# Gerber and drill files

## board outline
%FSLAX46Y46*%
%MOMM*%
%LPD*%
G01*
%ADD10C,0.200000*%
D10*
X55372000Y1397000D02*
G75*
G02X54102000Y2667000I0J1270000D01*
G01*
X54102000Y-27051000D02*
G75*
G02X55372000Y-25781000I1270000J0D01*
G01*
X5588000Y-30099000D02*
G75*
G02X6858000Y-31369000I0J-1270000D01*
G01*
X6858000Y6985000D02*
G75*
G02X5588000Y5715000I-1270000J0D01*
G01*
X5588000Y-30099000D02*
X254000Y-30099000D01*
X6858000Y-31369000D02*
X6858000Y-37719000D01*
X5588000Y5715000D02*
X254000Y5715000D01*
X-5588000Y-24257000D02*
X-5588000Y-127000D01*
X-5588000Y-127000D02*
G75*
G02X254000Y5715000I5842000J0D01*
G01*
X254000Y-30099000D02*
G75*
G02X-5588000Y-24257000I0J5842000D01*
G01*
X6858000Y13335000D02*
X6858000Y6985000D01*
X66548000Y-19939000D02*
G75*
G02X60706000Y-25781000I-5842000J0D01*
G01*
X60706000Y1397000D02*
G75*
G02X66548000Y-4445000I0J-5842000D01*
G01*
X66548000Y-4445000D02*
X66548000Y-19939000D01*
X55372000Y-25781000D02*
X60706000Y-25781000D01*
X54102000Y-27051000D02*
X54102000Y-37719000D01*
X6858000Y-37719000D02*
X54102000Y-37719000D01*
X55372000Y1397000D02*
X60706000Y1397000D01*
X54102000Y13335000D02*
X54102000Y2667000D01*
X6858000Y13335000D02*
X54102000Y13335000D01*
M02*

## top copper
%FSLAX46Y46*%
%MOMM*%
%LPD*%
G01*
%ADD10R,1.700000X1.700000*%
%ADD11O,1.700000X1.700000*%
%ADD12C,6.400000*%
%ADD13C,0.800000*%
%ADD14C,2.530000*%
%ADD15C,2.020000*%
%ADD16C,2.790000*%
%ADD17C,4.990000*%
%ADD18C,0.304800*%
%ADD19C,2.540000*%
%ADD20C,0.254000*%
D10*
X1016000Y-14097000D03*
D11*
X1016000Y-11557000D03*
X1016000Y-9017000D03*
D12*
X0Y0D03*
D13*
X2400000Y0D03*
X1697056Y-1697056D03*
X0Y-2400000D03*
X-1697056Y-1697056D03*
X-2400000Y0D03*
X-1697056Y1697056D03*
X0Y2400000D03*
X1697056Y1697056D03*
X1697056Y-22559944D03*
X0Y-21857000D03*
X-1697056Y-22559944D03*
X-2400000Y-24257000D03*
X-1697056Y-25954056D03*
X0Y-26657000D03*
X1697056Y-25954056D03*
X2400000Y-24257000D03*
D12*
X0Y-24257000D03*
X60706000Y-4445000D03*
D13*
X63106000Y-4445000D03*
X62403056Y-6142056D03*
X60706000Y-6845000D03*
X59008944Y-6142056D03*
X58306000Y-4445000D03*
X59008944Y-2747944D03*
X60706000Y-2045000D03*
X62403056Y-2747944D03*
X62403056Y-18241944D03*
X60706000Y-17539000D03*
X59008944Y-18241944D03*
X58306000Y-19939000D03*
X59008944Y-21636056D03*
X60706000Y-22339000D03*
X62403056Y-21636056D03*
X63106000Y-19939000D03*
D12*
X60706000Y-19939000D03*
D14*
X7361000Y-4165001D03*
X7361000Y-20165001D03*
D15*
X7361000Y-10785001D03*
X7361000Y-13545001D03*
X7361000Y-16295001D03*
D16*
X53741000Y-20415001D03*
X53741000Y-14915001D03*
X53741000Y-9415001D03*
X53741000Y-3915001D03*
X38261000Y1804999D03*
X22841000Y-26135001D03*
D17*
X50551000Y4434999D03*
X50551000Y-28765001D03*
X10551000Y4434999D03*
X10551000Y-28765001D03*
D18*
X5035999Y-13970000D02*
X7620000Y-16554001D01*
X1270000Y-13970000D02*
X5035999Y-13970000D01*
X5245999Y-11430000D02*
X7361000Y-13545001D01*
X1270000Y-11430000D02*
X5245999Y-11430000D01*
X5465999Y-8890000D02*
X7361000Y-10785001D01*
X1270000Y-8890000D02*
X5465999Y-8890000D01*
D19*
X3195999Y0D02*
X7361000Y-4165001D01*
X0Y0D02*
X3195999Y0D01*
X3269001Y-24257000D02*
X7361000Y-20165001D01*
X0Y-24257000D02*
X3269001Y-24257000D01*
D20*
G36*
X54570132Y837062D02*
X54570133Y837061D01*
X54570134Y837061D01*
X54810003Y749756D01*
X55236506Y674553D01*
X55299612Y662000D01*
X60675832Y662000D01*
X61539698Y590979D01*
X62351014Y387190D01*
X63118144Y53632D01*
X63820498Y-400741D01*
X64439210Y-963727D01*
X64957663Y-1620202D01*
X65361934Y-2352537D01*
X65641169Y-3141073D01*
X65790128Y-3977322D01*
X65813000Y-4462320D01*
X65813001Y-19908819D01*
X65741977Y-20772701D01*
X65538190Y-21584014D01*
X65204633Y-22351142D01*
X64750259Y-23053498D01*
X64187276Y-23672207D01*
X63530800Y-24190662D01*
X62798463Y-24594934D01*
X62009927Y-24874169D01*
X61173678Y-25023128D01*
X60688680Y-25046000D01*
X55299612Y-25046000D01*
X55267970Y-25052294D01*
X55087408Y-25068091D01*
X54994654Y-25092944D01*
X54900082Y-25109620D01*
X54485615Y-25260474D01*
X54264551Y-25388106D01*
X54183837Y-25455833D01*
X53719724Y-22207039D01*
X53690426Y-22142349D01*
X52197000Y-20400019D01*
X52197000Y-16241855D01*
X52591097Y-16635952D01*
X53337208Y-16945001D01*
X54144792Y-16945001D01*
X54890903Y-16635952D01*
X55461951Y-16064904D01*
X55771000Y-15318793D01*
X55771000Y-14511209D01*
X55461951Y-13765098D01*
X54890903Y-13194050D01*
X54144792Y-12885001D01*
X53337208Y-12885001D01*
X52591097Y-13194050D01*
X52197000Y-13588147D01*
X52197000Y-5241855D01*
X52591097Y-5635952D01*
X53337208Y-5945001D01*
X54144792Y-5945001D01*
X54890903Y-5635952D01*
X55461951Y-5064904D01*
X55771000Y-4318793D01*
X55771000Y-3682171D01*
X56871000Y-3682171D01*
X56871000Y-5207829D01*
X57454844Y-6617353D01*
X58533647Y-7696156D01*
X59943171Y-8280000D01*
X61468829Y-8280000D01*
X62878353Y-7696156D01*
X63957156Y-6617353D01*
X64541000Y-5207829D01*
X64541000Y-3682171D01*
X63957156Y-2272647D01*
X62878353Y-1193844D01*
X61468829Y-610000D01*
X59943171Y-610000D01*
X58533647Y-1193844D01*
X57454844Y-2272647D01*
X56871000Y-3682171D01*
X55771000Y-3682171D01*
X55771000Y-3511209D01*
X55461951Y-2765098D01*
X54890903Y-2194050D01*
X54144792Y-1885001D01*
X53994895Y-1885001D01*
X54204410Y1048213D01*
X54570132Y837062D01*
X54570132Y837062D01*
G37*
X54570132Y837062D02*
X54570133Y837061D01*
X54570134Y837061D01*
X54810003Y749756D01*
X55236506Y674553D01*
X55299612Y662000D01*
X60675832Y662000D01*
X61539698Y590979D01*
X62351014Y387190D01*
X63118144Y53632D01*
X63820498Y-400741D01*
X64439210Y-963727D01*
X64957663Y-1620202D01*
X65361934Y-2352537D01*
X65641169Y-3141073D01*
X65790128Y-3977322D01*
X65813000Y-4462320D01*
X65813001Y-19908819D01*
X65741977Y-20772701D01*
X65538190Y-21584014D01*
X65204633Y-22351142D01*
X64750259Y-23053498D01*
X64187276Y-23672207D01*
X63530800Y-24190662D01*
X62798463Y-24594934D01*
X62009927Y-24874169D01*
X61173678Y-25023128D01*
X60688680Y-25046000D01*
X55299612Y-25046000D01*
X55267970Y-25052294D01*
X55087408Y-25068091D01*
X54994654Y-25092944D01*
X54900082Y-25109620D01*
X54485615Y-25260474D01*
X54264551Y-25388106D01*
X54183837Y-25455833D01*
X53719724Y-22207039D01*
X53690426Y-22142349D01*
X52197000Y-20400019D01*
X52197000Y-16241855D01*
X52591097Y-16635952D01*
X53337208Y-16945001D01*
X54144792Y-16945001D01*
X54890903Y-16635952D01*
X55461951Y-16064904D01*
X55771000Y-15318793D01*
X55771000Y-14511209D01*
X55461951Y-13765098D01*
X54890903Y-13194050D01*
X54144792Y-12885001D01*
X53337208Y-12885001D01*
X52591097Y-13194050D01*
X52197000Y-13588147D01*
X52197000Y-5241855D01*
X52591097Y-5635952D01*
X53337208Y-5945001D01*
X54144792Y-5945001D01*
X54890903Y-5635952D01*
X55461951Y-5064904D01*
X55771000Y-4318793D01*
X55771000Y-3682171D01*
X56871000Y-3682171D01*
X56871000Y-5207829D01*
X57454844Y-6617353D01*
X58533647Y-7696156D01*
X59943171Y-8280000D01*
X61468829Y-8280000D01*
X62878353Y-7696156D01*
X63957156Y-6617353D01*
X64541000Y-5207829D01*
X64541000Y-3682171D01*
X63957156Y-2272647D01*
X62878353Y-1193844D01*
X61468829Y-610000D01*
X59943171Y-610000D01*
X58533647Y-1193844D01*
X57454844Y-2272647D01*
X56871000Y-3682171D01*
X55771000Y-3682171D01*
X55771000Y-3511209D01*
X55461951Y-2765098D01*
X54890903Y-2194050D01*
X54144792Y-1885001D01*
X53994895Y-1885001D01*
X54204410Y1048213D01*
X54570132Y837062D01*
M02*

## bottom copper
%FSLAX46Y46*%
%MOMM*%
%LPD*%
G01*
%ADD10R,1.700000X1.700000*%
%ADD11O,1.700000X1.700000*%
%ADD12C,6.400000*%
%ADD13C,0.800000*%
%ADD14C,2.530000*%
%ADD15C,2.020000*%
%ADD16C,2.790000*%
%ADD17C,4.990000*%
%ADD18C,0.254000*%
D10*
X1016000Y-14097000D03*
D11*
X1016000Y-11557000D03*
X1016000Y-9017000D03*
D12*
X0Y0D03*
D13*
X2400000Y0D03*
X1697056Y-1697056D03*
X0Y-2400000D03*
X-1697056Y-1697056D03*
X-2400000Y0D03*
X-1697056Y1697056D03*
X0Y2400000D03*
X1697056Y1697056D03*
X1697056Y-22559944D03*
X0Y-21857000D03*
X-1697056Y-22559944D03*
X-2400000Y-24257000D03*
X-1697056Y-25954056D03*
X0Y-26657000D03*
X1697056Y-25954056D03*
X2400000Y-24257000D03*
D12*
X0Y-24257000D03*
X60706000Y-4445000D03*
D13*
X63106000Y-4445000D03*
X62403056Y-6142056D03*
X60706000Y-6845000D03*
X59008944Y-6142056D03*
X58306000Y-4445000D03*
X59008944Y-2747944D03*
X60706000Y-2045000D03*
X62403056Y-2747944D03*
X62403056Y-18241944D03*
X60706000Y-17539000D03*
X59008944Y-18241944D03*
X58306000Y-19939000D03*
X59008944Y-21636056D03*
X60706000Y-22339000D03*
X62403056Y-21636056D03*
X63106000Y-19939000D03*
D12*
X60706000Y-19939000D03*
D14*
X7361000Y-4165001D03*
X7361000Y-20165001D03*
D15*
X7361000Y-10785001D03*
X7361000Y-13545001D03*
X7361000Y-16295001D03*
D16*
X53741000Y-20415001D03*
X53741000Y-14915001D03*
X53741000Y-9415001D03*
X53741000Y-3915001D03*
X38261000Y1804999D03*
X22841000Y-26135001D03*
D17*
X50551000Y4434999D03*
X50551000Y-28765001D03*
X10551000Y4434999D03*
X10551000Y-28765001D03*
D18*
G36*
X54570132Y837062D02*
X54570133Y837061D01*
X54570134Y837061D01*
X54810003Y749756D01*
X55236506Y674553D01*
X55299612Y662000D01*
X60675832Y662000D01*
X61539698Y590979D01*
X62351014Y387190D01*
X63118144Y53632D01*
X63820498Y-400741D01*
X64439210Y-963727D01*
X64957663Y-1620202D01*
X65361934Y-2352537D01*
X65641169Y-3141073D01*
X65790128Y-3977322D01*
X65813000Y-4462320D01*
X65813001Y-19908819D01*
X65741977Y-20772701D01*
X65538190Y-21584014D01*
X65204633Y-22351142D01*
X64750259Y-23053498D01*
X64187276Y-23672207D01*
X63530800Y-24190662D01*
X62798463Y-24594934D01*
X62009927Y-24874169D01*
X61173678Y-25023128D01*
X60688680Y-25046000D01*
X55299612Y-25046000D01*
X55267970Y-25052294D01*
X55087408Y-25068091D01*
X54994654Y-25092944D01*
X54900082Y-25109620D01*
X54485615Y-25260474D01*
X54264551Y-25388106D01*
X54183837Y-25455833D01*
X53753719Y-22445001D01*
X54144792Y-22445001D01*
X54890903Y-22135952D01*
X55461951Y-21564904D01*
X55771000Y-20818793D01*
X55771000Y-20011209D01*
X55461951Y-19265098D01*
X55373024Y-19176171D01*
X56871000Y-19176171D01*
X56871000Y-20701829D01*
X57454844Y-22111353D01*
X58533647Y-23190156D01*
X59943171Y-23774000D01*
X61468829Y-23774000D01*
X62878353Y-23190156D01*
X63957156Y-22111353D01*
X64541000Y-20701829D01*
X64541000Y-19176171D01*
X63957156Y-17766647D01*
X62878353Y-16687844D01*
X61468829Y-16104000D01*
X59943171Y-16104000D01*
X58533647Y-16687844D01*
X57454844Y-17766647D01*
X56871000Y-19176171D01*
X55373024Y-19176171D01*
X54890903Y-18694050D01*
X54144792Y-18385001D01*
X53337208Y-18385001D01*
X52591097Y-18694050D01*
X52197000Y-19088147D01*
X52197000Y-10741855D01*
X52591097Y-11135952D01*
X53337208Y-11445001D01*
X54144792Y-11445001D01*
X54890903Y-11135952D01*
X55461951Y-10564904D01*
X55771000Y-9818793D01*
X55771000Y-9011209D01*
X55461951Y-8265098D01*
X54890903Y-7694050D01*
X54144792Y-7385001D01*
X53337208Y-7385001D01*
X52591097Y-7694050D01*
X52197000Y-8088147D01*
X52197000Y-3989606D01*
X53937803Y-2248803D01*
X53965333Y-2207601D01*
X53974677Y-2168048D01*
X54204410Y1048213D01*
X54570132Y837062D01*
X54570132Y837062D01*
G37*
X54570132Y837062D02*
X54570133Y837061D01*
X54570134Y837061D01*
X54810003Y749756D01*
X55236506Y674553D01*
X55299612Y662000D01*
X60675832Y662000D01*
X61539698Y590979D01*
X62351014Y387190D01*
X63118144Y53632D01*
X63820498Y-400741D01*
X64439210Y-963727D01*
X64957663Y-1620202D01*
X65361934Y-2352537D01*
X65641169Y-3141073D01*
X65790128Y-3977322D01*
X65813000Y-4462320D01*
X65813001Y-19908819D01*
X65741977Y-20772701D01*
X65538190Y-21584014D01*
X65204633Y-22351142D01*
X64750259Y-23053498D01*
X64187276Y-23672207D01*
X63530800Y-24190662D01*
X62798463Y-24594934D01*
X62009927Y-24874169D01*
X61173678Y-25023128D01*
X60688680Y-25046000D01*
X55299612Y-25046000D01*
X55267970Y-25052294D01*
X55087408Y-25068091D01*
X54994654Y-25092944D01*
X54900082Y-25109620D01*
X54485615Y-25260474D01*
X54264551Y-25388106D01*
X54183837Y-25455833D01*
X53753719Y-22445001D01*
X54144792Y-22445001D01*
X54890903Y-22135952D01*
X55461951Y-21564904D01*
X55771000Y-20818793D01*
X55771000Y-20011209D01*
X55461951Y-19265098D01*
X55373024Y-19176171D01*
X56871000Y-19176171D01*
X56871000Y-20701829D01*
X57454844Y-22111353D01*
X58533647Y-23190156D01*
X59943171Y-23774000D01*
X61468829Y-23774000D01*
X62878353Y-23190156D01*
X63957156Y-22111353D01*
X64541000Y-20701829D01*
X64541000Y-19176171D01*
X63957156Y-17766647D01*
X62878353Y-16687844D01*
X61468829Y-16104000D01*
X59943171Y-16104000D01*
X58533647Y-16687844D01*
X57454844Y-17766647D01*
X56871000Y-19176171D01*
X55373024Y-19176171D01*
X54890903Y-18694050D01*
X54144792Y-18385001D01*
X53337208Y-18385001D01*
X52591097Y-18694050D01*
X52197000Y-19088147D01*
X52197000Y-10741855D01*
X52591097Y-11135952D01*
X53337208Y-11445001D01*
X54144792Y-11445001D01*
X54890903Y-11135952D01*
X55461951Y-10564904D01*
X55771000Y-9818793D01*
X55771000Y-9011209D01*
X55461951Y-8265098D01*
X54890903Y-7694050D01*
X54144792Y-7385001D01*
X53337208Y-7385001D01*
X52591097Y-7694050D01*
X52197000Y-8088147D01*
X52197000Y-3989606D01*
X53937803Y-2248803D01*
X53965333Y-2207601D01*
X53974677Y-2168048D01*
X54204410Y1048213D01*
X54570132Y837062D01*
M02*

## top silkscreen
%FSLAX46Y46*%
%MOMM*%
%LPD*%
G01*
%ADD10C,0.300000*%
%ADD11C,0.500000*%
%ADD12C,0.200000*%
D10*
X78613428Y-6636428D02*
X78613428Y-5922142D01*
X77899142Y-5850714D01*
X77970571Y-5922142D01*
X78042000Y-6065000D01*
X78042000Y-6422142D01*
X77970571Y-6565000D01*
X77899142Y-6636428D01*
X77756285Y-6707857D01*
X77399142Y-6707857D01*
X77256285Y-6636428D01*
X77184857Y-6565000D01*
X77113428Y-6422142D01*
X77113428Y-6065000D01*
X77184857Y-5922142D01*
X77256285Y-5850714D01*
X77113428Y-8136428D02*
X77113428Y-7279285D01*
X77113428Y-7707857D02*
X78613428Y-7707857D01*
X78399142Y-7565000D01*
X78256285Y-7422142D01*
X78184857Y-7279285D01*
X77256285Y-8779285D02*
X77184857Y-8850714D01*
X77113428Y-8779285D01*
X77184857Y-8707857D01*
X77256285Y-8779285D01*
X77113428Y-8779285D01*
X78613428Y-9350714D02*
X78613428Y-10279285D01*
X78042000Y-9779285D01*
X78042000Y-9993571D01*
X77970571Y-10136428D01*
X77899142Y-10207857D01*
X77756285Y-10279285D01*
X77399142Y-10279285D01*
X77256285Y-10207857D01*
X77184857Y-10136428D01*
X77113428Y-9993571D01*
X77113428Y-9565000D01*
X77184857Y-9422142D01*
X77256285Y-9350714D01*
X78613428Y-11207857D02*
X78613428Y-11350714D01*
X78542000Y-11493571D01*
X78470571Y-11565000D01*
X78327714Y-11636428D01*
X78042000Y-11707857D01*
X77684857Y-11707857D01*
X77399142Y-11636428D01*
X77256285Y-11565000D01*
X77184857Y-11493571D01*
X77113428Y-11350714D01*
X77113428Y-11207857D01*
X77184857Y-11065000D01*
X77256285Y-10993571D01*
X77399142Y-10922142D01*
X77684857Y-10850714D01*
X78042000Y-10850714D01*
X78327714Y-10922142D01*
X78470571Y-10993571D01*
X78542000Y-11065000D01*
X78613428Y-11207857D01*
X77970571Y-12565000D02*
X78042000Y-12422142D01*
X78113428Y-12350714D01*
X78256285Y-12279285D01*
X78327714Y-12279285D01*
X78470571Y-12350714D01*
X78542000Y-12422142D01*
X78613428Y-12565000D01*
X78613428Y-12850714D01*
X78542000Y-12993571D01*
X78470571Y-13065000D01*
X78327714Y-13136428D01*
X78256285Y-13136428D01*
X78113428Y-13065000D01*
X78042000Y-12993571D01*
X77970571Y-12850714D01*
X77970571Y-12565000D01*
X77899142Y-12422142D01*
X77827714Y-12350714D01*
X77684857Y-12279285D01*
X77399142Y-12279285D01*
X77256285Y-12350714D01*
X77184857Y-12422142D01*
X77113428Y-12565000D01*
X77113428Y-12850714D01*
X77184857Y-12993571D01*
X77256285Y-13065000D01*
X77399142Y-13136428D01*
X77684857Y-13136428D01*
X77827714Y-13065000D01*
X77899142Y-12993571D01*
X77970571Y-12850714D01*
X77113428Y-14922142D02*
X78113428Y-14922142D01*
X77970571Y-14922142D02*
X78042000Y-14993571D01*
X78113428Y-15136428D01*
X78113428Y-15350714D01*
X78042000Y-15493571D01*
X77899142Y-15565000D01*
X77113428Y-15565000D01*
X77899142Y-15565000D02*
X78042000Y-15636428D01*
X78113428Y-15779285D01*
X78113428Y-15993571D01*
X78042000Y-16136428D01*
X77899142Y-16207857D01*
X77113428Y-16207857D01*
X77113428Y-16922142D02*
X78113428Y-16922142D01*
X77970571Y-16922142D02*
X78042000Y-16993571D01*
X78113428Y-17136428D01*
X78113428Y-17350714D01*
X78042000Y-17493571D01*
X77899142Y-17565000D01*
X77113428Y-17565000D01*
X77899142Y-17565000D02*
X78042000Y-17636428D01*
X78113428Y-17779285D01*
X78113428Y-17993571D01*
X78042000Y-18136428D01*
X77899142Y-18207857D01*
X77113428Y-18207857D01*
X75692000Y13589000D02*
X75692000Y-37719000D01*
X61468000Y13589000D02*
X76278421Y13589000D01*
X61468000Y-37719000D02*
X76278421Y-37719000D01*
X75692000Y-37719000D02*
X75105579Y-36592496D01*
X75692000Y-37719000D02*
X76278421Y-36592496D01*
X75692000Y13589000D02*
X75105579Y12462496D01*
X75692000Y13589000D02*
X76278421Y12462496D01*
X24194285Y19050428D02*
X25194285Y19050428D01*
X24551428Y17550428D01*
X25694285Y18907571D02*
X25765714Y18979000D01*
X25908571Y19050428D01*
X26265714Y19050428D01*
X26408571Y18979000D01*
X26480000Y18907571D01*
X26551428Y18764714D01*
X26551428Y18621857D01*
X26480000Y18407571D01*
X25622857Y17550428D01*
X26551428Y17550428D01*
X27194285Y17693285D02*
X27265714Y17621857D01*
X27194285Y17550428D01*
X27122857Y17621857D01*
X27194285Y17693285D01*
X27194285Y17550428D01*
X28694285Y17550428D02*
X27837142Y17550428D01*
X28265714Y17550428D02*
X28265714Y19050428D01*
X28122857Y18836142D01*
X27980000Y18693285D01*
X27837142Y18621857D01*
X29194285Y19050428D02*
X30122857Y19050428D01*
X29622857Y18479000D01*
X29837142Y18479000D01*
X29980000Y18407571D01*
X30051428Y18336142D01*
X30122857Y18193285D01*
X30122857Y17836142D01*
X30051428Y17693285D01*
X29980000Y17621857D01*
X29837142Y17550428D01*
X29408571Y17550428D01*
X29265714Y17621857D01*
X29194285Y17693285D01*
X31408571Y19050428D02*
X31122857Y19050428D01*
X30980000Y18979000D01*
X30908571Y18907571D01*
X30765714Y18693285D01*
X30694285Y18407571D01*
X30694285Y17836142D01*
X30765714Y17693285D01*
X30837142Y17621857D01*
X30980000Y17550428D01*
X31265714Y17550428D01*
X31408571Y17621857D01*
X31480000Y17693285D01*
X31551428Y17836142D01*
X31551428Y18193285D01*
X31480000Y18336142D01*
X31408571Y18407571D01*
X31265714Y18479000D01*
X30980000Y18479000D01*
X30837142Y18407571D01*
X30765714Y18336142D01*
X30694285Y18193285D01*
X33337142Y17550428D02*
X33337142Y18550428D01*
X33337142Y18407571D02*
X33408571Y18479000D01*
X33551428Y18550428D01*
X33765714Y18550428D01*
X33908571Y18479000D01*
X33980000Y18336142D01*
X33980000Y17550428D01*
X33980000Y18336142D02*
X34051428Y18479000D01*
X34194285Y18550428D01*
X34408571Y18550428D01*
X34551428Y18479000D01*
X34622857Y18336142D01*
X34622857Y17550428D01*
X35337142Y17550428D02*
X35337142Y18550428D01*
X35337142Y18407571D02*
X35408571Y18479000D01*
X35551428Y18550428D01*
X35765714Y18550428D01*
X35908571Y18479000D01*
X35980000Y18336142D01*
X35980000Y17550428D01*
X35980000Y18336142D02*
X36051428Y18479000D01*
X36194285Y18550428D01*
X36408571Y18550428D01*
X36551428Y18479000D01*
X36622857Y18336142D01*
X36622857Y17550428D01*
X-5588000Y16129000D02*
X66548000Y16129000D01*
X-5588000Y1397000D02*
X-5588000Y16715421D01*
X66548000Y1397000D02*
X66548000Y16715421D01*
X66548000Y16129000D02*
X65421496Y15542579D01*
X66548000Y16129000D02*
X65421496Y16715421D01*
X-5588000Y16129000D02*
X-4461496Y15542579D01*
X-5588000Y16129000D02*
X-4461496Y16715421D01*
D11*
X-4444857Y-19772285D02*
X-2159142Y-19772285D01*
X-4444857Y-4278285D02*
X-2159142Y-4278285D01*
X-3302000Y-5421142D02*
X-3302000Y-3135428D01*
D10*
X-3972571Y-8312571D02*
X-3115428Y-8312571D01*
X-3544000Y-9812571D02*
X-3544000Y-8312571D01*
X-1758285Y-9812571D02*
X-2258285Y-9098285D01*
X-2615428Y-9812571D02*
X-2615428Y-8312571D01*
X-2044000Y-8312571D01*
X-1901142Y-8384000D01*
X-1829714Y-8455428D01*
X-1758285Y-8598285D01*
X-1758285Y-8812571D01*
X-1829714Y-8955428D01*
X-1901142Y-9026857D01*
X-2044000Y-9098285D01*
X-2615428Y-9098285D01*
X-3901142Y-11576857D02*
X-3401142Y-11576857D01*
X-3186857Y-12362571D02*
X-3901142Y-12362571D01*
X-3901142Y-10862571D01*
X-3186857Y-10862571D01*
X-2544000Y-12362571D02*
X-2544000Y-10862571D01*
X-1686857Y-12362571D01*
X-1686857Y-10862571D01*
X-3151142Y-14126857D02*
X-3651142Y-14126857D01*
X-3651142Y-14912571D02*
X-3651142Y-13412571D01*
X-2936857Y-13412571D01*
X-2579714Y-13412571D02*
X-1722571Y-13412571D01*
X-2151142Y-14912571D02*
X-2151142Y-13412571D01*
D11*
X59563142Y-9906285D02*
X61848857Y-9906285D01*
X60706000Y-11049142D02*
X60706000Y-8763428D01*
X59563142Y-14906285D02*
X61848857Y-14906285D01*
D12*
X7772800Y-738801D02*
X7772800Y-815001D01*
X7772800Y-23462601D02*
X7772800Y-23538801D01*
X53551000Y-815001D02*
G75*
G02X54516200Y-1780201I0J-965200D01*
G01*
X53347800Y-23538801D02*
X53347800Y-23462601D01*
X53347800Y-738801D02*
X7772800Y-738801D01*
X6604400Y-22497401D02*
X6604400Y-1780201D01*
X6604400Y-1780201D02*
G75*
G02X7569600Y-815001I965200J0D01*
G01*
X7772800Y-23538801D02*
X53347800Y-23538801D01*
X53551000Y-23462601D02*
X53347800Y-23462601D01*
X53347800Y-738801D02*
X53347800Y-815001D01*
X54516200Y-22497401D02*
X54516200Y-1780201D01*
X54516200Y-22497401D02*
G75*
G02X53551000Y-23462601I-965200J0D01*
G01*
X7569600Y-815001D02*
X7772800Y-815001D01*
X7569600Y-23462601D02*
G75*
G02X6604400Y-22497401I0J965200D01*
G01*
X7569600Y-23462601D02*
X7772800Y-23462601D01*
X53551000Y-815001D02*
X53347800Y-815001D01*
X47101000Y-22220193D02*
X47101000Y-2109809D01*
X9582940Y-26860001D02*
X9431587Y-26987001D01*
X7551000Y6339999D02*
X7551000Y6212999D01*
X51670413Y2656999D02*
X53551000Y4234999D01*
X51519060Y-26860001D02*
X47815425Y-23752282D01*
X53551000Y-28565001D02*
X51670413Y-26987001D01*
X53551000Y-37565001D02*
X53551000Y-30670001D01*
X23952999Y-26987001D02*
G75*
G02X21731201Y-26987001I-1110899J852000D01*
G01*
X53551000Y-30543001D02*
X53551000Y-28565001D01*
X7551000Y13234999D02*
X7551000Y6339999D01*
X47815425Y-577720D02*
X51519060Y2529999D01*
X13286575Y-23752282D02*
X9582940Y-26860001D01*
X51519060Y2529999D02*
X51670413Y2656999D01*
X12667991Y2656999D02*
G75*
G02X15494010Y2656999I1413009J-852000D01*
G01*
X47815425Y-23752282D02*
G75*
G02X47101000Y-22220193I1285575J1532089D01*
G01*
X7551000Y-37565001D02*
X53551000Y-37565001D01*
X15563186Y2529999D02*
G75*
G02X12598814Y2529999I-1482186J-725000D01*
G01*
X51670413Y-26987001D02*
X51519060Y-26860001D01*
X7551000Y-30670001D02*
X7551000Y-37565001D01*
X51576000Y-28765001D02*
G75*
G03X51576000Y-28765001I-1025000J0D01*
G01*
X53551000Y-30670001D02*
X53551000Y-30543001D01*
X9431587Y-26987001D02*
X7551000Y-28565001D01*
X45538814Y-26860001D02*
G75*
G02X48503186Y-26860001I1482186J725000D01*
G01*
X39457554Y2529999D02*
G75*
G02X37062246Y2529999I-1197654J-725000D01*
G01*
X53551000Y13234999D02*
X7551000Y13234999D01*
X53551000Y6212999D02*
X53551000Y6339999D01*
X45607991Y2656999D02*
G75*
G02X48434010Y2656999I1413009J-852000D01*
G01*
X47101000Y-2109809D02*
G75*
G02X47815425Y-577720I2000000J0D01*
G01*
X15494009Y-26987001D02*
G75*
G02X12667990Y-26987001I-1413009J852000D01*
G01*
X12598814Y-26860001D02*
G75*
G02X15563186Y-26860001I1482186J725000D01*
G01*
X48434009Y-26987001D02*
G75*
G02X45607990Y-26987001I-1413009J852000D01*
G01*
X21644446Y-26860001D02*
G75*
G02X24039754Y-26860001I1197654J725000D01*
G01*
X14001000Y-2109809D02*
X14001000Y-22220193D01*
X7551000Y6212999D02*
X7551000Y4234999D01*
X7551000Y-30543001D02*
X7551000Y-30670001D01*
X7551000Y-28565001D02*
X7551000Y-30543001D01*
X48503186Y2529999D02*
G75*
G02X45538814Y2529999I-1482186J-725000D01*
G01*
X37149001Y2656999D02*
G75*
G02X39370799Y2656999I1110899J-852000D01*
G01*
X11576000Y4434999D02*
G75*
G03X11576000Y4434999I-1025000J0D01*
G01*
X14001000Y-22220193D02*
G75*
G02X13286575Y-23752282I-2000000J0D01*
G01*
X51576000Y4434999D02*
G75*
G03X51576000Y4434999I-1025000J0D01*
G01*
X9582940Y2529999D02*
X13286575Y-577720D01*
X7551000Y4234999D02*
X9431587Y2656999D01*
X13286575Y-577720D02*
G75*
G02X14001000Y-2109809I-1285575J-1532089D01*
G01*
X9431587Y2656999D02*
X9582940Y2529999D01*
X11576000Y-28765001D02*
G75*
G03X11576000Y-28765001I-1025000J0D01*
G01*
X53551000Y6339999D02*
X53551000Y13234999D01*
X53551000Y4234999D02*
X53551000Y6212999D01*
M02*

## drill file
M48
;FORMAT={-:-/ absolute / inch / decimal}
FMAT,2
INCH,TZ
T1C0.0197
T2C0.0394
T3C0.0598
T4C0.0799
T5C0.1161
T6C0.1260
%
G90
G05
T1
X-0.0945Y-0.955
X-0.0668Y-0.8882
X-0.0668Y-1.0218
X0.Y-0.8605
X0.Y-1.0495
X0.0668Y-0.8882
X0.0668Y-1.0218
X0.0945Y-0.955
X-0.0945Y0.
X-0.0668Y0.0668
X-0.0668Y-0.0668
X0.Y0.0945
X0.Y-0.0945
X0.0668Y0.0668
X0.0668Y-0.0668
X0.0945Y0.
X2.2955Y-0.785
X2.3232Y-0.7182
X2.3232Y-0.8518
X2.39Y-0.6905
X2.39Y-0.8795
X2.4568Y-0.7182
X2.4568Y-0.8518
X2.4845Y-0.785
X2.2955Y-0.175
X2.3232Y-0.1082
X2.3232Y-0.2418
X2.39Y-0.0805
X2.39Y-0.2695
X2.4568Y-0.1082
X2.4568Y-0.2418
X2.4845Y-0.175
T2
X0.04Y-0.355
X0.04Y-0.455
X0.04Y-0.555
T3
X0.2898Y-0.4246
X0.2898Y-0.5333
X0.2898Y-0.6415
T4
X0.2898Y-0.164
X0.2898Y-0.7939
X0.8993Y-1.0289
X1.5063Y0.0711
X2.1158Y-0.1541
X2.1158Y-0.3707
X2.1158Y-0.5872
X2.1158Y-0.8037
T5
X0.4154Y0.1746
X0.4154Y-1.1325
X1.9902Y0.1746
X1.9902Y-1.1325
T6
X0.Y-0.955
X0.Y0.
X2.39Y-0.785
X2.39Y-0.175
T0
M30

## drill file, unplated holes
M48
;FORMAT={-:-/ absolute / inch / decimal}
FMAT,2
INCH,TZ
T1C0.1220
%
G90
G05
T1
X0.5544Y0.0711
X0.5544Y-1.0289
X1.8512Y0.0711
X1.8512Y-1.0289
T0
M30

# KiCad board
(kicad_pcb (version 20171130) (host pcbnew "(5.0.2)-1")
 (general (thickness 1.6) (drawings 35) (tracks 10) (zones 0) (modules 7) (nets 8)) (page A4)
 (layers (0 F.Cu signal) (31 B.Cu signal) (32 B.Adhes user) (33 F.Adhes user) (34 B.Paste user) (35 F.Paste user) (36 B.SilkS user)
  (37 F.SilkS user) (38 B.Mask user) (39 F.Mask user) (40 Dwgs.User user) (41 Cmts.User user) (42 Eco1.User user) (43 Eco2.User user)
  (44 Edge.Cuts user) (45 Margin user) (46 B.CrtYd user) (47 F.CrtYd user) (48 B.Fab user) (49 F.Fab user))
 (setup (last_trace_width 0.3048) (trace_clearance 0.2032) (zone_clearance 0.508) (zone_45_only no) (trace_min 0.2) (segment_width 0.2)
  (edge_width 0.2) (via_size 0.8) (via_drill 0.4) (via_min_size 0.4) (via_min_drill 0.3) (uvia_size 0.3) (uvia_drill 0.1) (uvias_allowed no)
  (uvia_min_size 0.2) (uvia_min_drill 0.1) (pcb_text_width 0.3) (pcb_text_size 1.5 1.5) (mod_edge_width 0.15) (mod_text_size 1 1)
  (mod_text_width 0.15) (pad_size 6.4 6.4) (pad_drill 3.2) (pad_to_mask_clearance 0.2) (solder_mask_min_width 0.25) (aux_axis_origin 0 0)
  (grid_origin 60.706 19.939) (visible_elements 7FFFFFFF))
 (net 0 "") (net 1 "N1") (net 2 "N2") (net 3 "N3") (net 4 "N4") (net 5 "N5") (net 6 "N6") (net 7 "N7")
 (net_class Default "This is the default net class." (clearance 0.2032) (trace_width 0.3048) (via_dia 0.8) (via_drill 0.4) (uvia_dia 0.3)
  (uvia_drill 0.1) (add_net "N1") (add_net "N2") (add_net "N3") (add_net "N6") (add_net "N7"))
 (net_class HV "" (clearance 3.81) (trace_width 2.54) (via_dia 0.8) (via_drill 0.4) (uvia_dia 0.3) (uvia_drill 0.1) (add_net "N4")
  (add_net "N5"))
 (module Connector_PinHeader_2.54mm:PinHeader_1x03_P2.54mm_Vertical (layer B.Cu) (at 1.016 14.097)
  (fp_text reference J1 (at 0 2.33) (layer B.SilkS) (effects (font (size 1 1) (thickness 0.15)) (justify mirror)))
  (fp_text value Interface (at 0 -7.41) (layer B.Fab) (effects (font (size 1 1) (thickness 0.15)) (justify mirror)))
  (pad 1 thru_hole rect (at 0 0) (size 1.7 1.7) (drill 1) (layers *.Cu *.Mask) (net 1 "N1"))
  (pad 2 thru_hole oval (at 0 -2.54) (size 1.7 1.7) (drill 1) (layers *.Cu *.Mask) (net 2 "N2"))
  (pad 3 thru_hole oval (at 0 -5.08) (size 1.7 1.7) (drill 1) (layers *.Cu *.Mask) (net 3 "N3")))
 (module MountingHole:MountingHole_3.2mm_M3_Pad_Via (layer F.Cu) (at 0 0)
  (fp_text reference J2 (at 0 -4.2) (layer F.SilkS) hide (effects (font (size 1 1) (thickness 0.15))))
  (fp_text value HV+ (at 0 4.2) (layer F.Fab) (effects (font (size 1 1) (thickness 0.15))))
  (pad 1 thru_hole circle (at 0 0) (size 6.4 6.4) (drill 3.2) (layers *.Cu *.Mask) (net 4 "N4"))
  (pad 1 thru_hole circle (at 2.4 0) (size 0.8 0.8) (drill 0.5) (layers *.Cu *.Mask) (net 4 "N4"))
  (pad 1 thru_hole circle (at 1.697056 1.697056) (size 0.8 0.8) (drill 0.5) (layers *.Cu *.Mask) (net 4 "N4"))
  (pad 1 thru_hole circle (at 0 2.4) (size 0.8 0.8) (drill 0.5) (layers *.Cu *.Mask) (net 4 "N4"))
  (pad 1 thru_hole circle (at -1.697056 1.697056) (size 0.8 0.8) (drill 0.5) (layers *.Cu *.Mask) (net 4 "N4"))
  (pad 1 thru_hole circle (at -2.4 0) (size 0.8 0.8) (drill 0.5) (layers *.Cu *.Mask) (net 4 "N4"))
  (pad 1 thru_hole circle (at -1.697056 -1.697056) (size 0.8 0.8) (drill 0.5) (layers *.Cu *.Mask) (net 4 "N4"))
  (pad 1 thru_hole circle (at 0 -2.4) (size 0.8 0.8) (drill 0.5) (layers *.Cu *.Mask) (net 4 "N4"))
  (pad 1 thru_hole circle (at 1.697056 -1.697056) (size 0.8 0.8) (drill 0.5) (layers *.Cu *.Mask) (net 4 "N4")))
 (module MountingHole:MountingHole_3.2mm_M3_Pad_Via (layer F.Cu) (at 0 24.257)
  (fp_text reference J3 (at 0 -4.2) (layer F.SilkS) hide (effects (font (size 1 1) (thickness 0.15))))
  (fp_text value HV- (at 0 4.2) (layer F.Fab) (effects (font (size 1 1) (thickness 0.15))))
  (pad 1 thru_hole circle (at 1.697056 -1.697056) (size 0.8 0.8) (drill 0.5) (layers *.Cu *.Mask) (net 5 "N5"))
  (pad 1 thru_hole circle (at 0 -2.4) (size 0.8 0.8) (drill 0.5) (layers *.Cu *.Mask) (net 5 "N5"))
  (pad 1 thru_hole circle (at -1.697056 -1.697056) (size 0.8 0.8) (drill 0.5) (layers *.Cu *.Mask) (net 5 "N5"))
  (pad 1 thru_hole circle (at -2.4 0) (size 0.8 0.8) (drill 0.5) (layers *.Cu *.Mask) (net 5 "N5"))
  (pad 1 thru_hole circle (at -1.697056 1.697056) (size 0.8 0.8) (drill 0.5) (layers *.Cu *.Mask) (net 5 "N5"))
  (pad 1 thru_hole circle (at 0 2.4) (size 0.8 0.8) (drill 0.5) (layers *.Cu *.Mask) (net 5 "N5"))
  (pad 1 thru_hole circle (at 1.697056 1.697056) (size 0.8 0.8) (drill 0.5) (layers *.Cu *.Mask) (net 5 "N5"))
  (pad 1 thru_hole circle (at 2.4 0) (size 0.8 0.8) (drill 0.5) (layers *.Cu *.Mask) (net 5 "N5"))
  (pad 1 thru_hole circle (at 0 0) (size 6.4 6.4) (drill 3.2) (layers *.Cu *.Mask) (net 5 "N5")))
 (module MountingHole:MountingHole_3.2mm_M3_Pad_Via (layer F.Cu) (at 60.706 4.445)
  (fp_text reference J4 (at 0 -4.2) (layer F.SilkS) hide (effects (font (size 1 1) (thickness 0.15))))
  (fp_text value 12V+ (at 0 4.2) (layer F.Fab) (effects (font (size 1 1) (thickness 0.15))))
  (pad 1 thru_hole circle (at 0 0) (size 6.4 6.4) (drill 3.2) (layers *.Cu *.Mask) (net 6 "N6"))
  (pad 1 thru_hole circle (at 2.4 0) (size 0.8 0.8) (drill 0.5) (layers *.Cu *.Mask) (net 6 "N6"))
  (pad 1 thru_hole circle (at 1.697056 1.697056) (size 0.8 0.8) (drill 0.5) (layers *.Cu *.Mask) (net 6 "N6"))
  (pad 1 thru_hole circle (at 0 2.4) (size 0.8 0.8) (drill 0.5) (layers *.Cu *.Mask) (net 6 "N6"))
  (pad 1 thru_hole circle (at -1.697056 1.697056) (size 0.8 0.8) (drill 0.5) (layers *.Cu *.Mask) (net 6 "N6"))
  (pad 1 thru_hole circle (at -2.4 0) (size 0.8 0.8) (drill 0.5) (layers *.Cu *.Mask) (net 6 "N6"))
  (pad 1 thru_hole circle (at -1.697056 -1.697056) (size 0.8 0.8) (drill 0.5) (layers *.Cu *.Mask) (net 6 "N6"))
  (pad 1 thru_hole circle (at 0 -2.4) (size 0.8 0.8) (drill 0.5) (layers *.Cu *.Mask) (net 6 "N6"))
  (pad 1 thru_hole circle (at 1.697056 -1.697056) (size 0.8 0.8) (drill 0.5) (layers *.Cu *.Mask) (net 6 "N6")))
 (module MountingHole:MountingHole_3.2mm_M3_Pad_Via (layer F.Cu) (at 60.706 19.939)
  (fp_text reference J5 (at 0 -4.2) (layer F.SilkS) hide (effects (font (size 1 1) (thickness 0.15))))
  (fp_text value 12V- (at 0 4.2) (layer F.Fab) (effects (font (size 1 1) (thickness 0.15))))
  (pad 1 thru_hole circle (at 1.697056 -1.697056) (size 0.8 0.8) (drill 0.5) (layers *.Cu *.Mask) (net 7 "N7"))
  (pad 1 thru_hole circle (at 0 -2.4) (size 0.8 0.8) (drill 0.5) (layers *.Cu *.Mask) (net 7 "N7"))
  (pad 1 thru_hole circle (at -1.697056 -1.697056) (size 0.8 0.8) (drill 0.5) (layers *.Cu *.Mask) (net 7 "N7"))
  (pad 1 thru_hole circle (at -2.4 0) (size 0.8 0.8) (drill 0.5) (layers *.Cu *.Mask) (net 7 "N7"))
  (pad 1 thru_hole circle (at -1.697056 1.697056) (size 0.8 0.8) (drill 0.5) (layers *.Cu *.Mask) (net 7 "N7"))
  (pad 1 thru_hole circle (at 0 2.4) (size 0.8 0.8) (drill 0.5) (layers *.Cu *.Mask) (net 7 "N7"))
  (pad 1 thru_hole circle (at 1.697056 1.697056) (size 0.8 0.8) (drill 0.5) (layers *.Cu *.Mask) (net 7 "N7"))
  (pad 1 thru_hole circle (at 2.4 0) (size 0.8 0.8) (drill 0.5) (layers *.Cu *.Mask) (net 7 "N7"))
  (pad 1 thru_hole circle (at 0 0) (size 6.4 6.4) (drill 3.2) (layers *.Cu *.Mask) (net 7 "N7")))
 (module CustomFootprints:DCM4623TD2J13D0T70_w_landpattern (layer F.Cu) (at 30.551 12.165001)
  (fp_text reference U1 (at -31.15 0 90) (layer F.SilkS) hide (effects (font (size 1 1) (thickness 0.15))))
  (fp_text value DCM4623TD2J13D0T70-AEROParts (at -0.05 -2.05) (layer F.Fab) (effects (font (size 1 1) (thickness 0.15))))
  (fp_line (start -22.7782 -11.4262) (end -22.7782 -11.35) (layer F.SilkS) (width 0.2))
  (fp_line (start -22.7782 11.2976) (end -22.7782 11.3738) (layer F.SilkS) (width 0.2))
  (fp_arc (start 23 -10.3848) (end 23.9652 -10.3848) (angle -90) (layer F.SilkS) (width 0.2))
  (fp_line (start 22.7968 11.3738) (end 22.7968 11.2976) (layer F.SilkS) (width 0.2))
  (fp_line (start 22.7968 -11.4262) (end -22.7782 -11.4262) (layer F.SilkS) (width 0.2))
  (fp_line (start -23.9466 10.3324) (end -23.9466 -10.3848) (layer F.SilkS) (width 0.2))
  (fp_arc (start -22.9814 -10.3848) (end -22.9814 -11.35) (angle -90) (layer F.SilkS) (width 0.2))
  (fp_line (start -22.7782 11.3738) (end 22.7968 11.3738) (layer F.SilkS) (width 0.2))
  (fp_line (start 23 11.2976) (end 22.7968 11.2976) (layer F.SilkS) (width 0.2))
  (fp_line (start 22.7968 -11.4262) (end 22.7968 -11.35) (layer F.SilkS) (width 0.2))
  (fp_line (start 23.9652 10.3324) (end 23.9652 -10.3848) (layer F.SilkS) (width 0.2))
  (fp_arc (start 23 10.3324) (end 23 11.2976) (angle -90) (layer F.SilkS) (width 0.2))
  (fp_line (start -22.9814 -11.35) (end -22.7782 -11.35) (layer F.SilkS) (width 0.2))
  (fp_arc (start -22.9814 10.3324) (end -23.9466 10.3324) (angle -90) (layer F.SilkS) (width 0.2))
  (fp_line (start -22.9814 11.2976) (end -22.7782 11.2976) (layer F.SilkS) (width 0.2))
  (fp_line (start 23 -11.35) (end 22.7968 -11.35) (layer F.SilkS) (width 0.2))
  (fp_line (start 16.55 10.055192) (end 16.55 -10.055192) (layer F.SilkS) (width 0.2))
  (fp_line (start -20.96806 14.695) (end -21.119413 14.822) (layer F.SilkS) (width 0.2))
  (fp_line (start -23 -18.505) (end -23 -18.378) (layer F.SilkS) (width 0.2))
  (fp_line (start 21.119413 -14.822) (end 23 -16.4) (layer F.SilkS) (width 0.2))
  (fp_line (start 20.96806 14.695) (end 17.264425 11.587281) (layer F.SilkS) (width 0.2))
  (fp_line (start 23 16.4) (end 21.119413 14.822) (layer F.SilkS) (width 0.2))
  (fp_line (start 23 25.4) (end 23 18.505) (layer F.SilkS) (width 0.2))
  (fp_arc (start -7.7089 13.97) (end -8.819799 14.822) (angle -105.0274407) (layer F.SilkS) (width 0.2))
  (fp_line (start 23 18.378) (end 23 16.4) (layer F.SilkS) (width 0.2))
  (fp_line (start -23 -25.4) (end -23 -18.505) (layer F.SilkS) (width 0.2))
  (fp_line (start 17.264425 -11.587281) (end 20.96806 -14.695) (layer F.SilkS) (width 0.2))
  (fp_line (start -17.264425 11.587281) (end -20.96806 14.695) (layer F.SilkS) (width 0.2))
  (fp_line (start 20.96806 -14.695) (end 21.119413 -14.822) (layer F.SilkS) (width 0.2))
  (fp_arc (start -16.47 -13.97) (end -15.05699 -14.822) (angle -117.8227081) (layer F.SilkS) (width 0.2))
  (fp_arc (start 18.55 10.055192) (end 16.55 10.055192) (angle -50) (layer F.SilkS) (width 0.2))
  (fp_line (start -23 25.4) (end 23 25.4) (layer F.SilkS) (width 0.2))
  (fp_arc (start -16.47 -13.97) (end -17.952186 -14.695) (angle -232.130437) (layer F.SilkS) (width 0.2))
  (fp_line (start 21.119413 14.822) (end 20.96806 14.695) (layer F.SilkS) (width 0.2))
  (fp_line (start -23 18.505) (end -23 25.4) (layer F.SilkS) (width 0.2))
  (fp_circle (center 20 16.6) (end 20 15.575) (layer F.SilkS) (width 0.2))
  (fp_line (start 23 18.505) (end 23 18.378) (layer F.SilkS) (width 0.2))
  (fp_line (start -21.119413 14.822) (end -23 16.4) (layer F.SilkS) (width 0.2))
  (fp_arc (start 16.47 13.97) (end 17.952186 14.695) (angle -232.130437) (layer F.SilkS) (width 0.2))
  (fp_arc (start 7.7089 -13.97) (end 6.511246 -14.695) (angle -242.377245) (layer F.SilkS) (width 0.2))
  (fp_line (start 23 -25.4) (end -23 -25.4) (layer F.SilkS) (width 0.2))
  (fp_line (start 23 -18.378) (end 23 -18.505) (layer F.SilkS) (width 0.2))
  (fp_arc (start 16.47 -13.97) (end 17.88301 -14.822) (angle -117.8227081) (layer F.SilkS) (width 0.2))
  (fp_arc (start 18.55 -10.055192) (end 17.264425 -11.587281) (angle -50) (layer F.SilkS) (width 0.2))
  (fp_arc (start -16.47 13.97) (end -17.88301 14.822) (angle -117.8227081) (layer F.SilkS) (width 0.2))
  (fp_arc (start -16.47 13.97) (end -14.987814 14.695) (angle -232.130437) (layer F.SilkS) (width 0.2))
  (fp_arc (start 16.47 13.97) (end 15.05699 14.822) (angle -117.8227081) (layer F.SilkS) (width 0.2))
  (fp_arc (start -7.7089 13.97) (end -6.511246 14.695) (angle -242.377245) (layer F.SilkS) (width 0.2))
  (fp_line (start -16.55 -10.055192) (end -16.55 10.055192) (layer F.SilkS) (width 0.2))
  (fp_line (start -23 -18.378) (end -23 -16.4) (layer F.SilkS) (width 0.2))
  (fp_line (start -23 18.378) (end -23 18.505) (layer F.SilkS) (width 0.2))
  (fp_line (start -23 16.4) (end -23 18.378) (layer F.SilkS) (width 0.2))
  (fp_arc (start 16.47 -13.97) (end 14.987814 -14.695) (angle -232.130437) (layer F.SilkS) (width 0.2))
  (fp_arc (start 7.7089 -13.97) (end 8.819799 -14.822) (angle -105.0274407) (layer F.SilkS) (width 0.2))
  (fp_circle (center -20 -16.6) (end -20 -17.625) (layer F.SilkS) (width 0.2))
  (fp_arc (start -18.55 10.055192) (end -17.264425 11.587281) (angle -50) (layer F.SilkS) (width 0.2))
  (fp_circle (center 20 -16.6) (end 20 -17.625) (layer F.SilkS) (width 0.2))
  (fp_line (start -20.96806 -14.695) (end -17.264425 -11.587281) (layer F.SilkS) (width 0.2))
  (fp_line (start -23 -16.4) (end -21.119413 -14.822) (layer F.SilkS) (width 0.2))
  (fp_arc (start -18.55 -10.055192) (end -16.55 -10.055192) (angle -50) (layer F.SilkS) (width 0.2))
  (fp_line (start -21.119413 -14.822) (end -20.96806 -14.695) (layer F.SilkS) (width 0.2))
  (fp_circle (center -20 16.6) (end -20 15.575) (layer F.SilkS) (width 0.2))
  (fp_line (start 23 -18.505) (end 23 -25.4) (layer F.SilkS) (width 0.2))
  (fp_line (start 23 -16.4) (end 23 -18.378) (layer F.SilkS) (width 0.2))
  (pad 1 thru_hole circle (at -23.19 -8) (size 2.53 2.53) (drill 2.03) (layers *.Cu *.Mask) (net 4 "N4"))
  (pad 5 thru_hole circle (at -23.19 8) (size 2.53 2.53) (drill 2.03) (layers *.Cu *.Mask) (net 5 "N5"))
  (pad 2 thru_hole circle (at -23.19 -1.38) (size 2.02 2.02) (drill 1.52) (layers *.Cu *.Mask) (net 3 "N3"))
  (pad 3 thru_hole circle (at -23.19 1.38) (size 2.02 2.02) (drill 1.52) (layers *.Cu *.Mask) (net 2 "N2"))
  (pad 4 thru_hole circle (at -23.19 4.13) (size 2.02 2.02) (drill 1.52) (layers *.Cu *.Mask) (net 1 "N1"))
  (pad 6 thru_hole circle (at 23.19 8.25) (size 2.79 2.79) (drill 2.03) (layers *.Cu *.Mask) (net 7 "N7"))
  (pad 7 thru_hole circle (at 23.19 2.75) (size 2.79 2.79) (drill 2.03) (layers *.Cu *.Mask) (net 6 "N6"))
  (pad 8 thru_hole circle (at 23.19 -2.75) (size 2.79 2.79) (drill 2.03) (layers *.Cu *.Mask) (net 7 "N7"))
  (pad 9 thru_hole circle (at 23.19 -8.25) (size 2.79 2.79) (drill 2.03) (layers *.Cu *.Mask) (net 6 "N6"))
  (pad "" np_thru_hole circle (at 16.47 -13.97) (size 3.1 3.1) (drill 3.1) (layers *.Cu *.Mask))
  (pad "" np_thru_hole circle (at -16.47 -13.97) (size 3.1 3.1) (drill 3.1) (layers *.Cu *.Mask))
  (pad "" np_thru_hole circle (at -16.47 13.97) (size 3.1 3.1) (drill 3.1) (layers *.Cu *.Mask))
  (pad "" np_thru_hole circle (at 16.47 13.97) (size 3.1 3.1) (drill 3.1) (layers *.Cu *.Mask))
  (pad "" thru_hole circle (at 7.71 -13.97) (size 2.79 2.79) (drill 2.03) (layers *.Cu *.Mask))
  (pad "" thru_hole circle (at -7.71 13.97) (size 2.79 2.79) (drill 2.03) (layers *.Cu *.Mask))
  (pad "" thru_hole circle (at 20 -16.6) (size 4.99 4.99) (drill 2.95) (layers *.Cu *.Mask))
  (pad "" thru_hole circle (at 20 16.6) (size 4.99 4.99) (drill 2.95) (layers *.Cu *.Mask))
  (pad "" thru_hole circle (at -20 -16.6) (size 4.99 4.99) (drill 2.95) (layers *.Cu *.Mask))
  (pad "" thru_hole circle (at -20 16.6) (size 4.99 4.99) (drill 2.95) (layers *.Cu *.Mask)))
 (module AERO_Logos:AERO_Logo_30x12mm (layer B.Cu) (at 30.988 11.43 180)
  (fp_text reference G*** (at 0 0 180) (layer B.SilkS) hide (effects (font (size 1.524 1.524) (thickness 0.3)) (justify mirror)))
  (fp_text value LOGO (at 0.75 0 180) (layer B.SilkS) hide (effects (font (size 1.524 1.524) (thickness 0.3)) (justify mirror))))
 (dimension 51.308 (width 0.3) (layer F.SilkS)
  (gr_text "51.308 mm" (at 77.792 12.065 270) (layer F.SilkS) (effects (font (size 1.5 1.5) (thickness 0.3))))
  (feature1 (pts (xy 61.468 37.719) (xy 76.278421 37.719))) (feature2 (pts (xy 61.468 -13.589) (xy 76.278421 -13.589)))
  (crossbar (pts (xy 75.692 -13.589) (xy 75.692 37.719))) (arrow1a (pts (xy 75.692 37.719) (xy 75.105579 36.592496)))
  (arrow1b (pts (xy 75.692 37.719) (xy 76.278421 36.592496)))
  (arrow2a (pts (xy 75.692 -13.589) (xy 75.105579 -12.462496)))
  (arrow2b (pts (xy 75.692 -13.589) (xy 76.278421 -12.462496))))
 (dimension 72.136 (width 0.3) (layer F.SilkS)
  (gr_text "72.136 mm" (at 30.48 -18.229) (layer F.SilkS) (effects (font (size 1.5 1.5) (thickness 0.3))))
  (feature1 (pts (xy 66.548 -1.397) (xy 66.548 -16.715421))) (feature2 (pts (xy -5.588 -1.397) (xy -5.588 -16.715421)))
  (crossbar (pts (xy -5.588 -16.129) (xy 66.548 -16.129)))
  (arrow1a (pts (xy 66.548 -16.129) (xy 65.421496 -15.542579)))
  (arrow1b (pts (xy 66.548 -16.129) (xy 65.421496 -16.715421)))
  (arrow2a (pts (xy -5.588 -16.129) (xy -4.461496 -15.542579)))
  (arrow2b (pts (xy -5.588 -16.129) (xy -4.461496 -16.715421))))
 (gr_arc (start 55.372 -2.667) (end 54.102 -2.667) (angle -90) (layer Edge.Cuts) (width 0.2))
 (gr_arc (start 55.372 27.051) (end 55.372 25.781) (angle -90) (layer Edge.Cuts) (width 0.2))
 (gr_arc (start 5.588 31.369) (end 6.858 31.369) (angle -90) (layer Edge.Cuts) (width 0.2))
 (gr_arc (start 5.588 -6.985) (end 5.588 -5.715) (angle -90) (layer Edge.Cuts) (width 0.2))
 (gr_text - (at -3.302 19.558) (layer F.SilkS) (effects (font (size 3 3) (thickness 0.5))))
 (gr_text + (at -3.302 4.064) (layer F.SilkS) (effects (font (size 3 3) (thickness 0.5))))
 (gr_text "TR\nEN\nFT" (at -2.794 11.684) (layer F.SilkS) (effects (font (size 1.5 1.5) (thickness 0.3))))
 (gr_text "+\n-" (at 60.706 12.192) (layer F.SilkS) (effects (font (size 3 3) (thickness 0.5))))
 (gr_line (start 5.588 30.099) (end 0.254 30.099) (layer Edge.Cuts) (width 0.2))
 (gr_line (start 6.858 31.369) (end 6.858 37.719) (layer Edge.Cuts) (width 0.2))
 (gr_line (start 5.588 -5.715) (end 0.254 -5.715) (layer Edge.Cuts) (width 0.2))
 (gr_line (start -5.588 24.257) (end -5.588 0.127) (layer Edge.Cuts) (width 0.2))
 (gr_arc (start 0.254 0.127) (end 0.254 -5.715) (angle -90) (layer Edge.Cuts) (width 0.2))
 (gr_arc (start 0.254 24.257) (end -5.588 24.257) (angle -90) (layer Edge.Cuts) (width 0.2))
 (gr_line (start 6.858 -13.335) (end 6.858 -6.985) (layer Edge.Cuts) (width 0.2))
 (gr_arc (start 60.706 19.939) (end 60.706 25.781) (angle -90) (layer Edge.Cuts) (width 0.2))
 (gr_arc (start 60.706 4.445) (end 66.548 4.445) (angle -90) (layer Edge.Cuts) (width 0.2))
 (gr_line (start 66.548 4.445) (end 66.548 19.939) (layer Edge.Cuts) (width 0.2))
 (gr_line (start 55.372 25.781) (end 60.706 25.781) (layer Edge.Cuts) (width 0.2))
 (gr_line (start 54.102 27.051) (end 54.102 37.719) (layer Edge.Cuts) (width 0.2))
 (gr_line (start 6.858 37.719) (end 54.102 37.719) (layer Edge.Cuts) (width 0.2))
 (gr_line (start 55.372 -1.397) (end 60.706 -1.397) (layer Edge.Cuts) (width 0.2))
 (gr_line (start 54.102 -13.335) (end 54.102 -2.667) (layer Edge.Cuts) (width 0.2))
 (gr_line (start 6.858 -13.335) (end 54.102 -13.335) (layer Edge.Cuts) (width 0.2))
 (segment (start 5.035999 13.97) (end 7.62 16.554001) (width 0.3048) (layer F.Cu) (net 1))
 (segment (start 1.27 13.97) (end 5.035999 13.97) (width 0.3048) (layer F.Cu) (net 1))
 (segment (start 5.245999 11.43) (end 7.361 13.545001) (width 0.3048) (layer F.Cu) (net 2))
 (segment (start 1.27 11.43) (end 5.245999 11.43) (width 0.3048) (layer F.Cu) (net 2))
 (segment (start 5.465999 8.89) (end 7.361 10.785001) (width 0.3048) (layer F.Cu) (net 3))
 (segment (start 1.27 8.89) (end 5.465999 8.89) (width 0.3048) (layer F.Cu) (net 3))
 (segment (start 3.195999 0) (end 7.361 4.165001) (width 2.54) (layer F.Cu) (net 4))
 (segment (start 0 0) (end 3.195999 0) (width 2.54) (layer F.Cu) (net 4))
 (segment (start 3.269001 24.257) (end 7.361 20.165001) (width 2.54) (layer F.Cu) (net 5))
 (segment (start 0 24.257) (end 3.269001 24.257) (width 2.54) (layer F.Cu) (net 5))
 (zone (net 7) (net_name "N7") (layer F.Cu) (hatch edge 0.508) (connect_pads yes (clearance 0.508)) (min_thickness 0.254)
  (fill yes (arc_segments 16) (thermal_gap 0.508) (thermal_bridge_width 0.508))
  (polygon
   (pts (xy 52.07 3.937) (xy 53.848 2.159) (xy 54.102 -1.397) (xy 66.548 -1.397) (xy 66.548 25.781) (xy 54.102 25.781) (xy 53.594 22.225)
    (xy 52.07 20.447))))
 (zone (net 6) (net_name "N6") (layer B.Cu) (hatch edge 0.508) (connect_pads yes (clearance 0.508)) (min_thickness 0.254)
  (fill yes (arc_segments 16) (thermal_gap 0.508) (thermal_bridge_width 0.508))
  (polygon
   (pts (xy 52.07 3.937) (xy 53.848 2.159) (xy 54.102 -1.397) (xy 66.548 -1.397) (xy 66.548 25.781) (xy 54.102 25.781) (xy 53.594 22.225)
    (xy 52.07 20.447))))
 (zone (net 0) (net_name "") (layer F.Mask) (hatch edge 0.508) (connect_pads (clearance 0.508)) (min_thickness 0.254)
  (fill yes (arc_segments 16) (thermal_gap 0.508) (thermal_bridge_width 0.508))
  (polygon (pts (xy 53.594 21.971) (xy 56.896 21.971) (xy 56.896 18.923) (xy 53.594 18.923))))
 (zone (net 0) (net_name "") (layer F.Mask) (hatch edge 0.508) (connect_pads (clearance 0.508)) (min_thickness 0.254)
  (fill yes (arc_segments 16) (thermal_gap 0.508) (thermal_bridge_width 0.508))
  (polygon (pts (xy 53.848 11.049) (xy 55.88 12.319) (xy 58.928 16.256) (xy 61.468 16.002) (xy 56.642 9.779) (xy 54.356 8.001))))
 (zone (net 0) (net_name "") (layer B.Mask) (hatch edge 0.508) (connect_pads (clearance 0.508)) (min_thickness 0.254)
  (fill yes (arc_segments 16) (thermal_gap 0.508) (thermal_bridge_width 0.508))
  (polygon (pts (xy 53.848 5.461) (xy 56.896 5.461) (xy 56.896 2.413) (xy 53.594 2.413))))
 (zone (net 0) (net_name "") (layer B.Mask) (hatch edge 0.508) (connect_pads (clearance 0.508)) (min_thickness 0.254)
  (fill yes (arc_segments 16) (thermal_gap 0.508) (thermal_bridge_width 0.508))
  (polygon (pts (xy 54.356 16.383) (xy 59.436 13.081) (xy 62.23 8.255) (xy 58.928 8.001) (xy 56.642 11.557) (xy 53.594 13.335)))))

